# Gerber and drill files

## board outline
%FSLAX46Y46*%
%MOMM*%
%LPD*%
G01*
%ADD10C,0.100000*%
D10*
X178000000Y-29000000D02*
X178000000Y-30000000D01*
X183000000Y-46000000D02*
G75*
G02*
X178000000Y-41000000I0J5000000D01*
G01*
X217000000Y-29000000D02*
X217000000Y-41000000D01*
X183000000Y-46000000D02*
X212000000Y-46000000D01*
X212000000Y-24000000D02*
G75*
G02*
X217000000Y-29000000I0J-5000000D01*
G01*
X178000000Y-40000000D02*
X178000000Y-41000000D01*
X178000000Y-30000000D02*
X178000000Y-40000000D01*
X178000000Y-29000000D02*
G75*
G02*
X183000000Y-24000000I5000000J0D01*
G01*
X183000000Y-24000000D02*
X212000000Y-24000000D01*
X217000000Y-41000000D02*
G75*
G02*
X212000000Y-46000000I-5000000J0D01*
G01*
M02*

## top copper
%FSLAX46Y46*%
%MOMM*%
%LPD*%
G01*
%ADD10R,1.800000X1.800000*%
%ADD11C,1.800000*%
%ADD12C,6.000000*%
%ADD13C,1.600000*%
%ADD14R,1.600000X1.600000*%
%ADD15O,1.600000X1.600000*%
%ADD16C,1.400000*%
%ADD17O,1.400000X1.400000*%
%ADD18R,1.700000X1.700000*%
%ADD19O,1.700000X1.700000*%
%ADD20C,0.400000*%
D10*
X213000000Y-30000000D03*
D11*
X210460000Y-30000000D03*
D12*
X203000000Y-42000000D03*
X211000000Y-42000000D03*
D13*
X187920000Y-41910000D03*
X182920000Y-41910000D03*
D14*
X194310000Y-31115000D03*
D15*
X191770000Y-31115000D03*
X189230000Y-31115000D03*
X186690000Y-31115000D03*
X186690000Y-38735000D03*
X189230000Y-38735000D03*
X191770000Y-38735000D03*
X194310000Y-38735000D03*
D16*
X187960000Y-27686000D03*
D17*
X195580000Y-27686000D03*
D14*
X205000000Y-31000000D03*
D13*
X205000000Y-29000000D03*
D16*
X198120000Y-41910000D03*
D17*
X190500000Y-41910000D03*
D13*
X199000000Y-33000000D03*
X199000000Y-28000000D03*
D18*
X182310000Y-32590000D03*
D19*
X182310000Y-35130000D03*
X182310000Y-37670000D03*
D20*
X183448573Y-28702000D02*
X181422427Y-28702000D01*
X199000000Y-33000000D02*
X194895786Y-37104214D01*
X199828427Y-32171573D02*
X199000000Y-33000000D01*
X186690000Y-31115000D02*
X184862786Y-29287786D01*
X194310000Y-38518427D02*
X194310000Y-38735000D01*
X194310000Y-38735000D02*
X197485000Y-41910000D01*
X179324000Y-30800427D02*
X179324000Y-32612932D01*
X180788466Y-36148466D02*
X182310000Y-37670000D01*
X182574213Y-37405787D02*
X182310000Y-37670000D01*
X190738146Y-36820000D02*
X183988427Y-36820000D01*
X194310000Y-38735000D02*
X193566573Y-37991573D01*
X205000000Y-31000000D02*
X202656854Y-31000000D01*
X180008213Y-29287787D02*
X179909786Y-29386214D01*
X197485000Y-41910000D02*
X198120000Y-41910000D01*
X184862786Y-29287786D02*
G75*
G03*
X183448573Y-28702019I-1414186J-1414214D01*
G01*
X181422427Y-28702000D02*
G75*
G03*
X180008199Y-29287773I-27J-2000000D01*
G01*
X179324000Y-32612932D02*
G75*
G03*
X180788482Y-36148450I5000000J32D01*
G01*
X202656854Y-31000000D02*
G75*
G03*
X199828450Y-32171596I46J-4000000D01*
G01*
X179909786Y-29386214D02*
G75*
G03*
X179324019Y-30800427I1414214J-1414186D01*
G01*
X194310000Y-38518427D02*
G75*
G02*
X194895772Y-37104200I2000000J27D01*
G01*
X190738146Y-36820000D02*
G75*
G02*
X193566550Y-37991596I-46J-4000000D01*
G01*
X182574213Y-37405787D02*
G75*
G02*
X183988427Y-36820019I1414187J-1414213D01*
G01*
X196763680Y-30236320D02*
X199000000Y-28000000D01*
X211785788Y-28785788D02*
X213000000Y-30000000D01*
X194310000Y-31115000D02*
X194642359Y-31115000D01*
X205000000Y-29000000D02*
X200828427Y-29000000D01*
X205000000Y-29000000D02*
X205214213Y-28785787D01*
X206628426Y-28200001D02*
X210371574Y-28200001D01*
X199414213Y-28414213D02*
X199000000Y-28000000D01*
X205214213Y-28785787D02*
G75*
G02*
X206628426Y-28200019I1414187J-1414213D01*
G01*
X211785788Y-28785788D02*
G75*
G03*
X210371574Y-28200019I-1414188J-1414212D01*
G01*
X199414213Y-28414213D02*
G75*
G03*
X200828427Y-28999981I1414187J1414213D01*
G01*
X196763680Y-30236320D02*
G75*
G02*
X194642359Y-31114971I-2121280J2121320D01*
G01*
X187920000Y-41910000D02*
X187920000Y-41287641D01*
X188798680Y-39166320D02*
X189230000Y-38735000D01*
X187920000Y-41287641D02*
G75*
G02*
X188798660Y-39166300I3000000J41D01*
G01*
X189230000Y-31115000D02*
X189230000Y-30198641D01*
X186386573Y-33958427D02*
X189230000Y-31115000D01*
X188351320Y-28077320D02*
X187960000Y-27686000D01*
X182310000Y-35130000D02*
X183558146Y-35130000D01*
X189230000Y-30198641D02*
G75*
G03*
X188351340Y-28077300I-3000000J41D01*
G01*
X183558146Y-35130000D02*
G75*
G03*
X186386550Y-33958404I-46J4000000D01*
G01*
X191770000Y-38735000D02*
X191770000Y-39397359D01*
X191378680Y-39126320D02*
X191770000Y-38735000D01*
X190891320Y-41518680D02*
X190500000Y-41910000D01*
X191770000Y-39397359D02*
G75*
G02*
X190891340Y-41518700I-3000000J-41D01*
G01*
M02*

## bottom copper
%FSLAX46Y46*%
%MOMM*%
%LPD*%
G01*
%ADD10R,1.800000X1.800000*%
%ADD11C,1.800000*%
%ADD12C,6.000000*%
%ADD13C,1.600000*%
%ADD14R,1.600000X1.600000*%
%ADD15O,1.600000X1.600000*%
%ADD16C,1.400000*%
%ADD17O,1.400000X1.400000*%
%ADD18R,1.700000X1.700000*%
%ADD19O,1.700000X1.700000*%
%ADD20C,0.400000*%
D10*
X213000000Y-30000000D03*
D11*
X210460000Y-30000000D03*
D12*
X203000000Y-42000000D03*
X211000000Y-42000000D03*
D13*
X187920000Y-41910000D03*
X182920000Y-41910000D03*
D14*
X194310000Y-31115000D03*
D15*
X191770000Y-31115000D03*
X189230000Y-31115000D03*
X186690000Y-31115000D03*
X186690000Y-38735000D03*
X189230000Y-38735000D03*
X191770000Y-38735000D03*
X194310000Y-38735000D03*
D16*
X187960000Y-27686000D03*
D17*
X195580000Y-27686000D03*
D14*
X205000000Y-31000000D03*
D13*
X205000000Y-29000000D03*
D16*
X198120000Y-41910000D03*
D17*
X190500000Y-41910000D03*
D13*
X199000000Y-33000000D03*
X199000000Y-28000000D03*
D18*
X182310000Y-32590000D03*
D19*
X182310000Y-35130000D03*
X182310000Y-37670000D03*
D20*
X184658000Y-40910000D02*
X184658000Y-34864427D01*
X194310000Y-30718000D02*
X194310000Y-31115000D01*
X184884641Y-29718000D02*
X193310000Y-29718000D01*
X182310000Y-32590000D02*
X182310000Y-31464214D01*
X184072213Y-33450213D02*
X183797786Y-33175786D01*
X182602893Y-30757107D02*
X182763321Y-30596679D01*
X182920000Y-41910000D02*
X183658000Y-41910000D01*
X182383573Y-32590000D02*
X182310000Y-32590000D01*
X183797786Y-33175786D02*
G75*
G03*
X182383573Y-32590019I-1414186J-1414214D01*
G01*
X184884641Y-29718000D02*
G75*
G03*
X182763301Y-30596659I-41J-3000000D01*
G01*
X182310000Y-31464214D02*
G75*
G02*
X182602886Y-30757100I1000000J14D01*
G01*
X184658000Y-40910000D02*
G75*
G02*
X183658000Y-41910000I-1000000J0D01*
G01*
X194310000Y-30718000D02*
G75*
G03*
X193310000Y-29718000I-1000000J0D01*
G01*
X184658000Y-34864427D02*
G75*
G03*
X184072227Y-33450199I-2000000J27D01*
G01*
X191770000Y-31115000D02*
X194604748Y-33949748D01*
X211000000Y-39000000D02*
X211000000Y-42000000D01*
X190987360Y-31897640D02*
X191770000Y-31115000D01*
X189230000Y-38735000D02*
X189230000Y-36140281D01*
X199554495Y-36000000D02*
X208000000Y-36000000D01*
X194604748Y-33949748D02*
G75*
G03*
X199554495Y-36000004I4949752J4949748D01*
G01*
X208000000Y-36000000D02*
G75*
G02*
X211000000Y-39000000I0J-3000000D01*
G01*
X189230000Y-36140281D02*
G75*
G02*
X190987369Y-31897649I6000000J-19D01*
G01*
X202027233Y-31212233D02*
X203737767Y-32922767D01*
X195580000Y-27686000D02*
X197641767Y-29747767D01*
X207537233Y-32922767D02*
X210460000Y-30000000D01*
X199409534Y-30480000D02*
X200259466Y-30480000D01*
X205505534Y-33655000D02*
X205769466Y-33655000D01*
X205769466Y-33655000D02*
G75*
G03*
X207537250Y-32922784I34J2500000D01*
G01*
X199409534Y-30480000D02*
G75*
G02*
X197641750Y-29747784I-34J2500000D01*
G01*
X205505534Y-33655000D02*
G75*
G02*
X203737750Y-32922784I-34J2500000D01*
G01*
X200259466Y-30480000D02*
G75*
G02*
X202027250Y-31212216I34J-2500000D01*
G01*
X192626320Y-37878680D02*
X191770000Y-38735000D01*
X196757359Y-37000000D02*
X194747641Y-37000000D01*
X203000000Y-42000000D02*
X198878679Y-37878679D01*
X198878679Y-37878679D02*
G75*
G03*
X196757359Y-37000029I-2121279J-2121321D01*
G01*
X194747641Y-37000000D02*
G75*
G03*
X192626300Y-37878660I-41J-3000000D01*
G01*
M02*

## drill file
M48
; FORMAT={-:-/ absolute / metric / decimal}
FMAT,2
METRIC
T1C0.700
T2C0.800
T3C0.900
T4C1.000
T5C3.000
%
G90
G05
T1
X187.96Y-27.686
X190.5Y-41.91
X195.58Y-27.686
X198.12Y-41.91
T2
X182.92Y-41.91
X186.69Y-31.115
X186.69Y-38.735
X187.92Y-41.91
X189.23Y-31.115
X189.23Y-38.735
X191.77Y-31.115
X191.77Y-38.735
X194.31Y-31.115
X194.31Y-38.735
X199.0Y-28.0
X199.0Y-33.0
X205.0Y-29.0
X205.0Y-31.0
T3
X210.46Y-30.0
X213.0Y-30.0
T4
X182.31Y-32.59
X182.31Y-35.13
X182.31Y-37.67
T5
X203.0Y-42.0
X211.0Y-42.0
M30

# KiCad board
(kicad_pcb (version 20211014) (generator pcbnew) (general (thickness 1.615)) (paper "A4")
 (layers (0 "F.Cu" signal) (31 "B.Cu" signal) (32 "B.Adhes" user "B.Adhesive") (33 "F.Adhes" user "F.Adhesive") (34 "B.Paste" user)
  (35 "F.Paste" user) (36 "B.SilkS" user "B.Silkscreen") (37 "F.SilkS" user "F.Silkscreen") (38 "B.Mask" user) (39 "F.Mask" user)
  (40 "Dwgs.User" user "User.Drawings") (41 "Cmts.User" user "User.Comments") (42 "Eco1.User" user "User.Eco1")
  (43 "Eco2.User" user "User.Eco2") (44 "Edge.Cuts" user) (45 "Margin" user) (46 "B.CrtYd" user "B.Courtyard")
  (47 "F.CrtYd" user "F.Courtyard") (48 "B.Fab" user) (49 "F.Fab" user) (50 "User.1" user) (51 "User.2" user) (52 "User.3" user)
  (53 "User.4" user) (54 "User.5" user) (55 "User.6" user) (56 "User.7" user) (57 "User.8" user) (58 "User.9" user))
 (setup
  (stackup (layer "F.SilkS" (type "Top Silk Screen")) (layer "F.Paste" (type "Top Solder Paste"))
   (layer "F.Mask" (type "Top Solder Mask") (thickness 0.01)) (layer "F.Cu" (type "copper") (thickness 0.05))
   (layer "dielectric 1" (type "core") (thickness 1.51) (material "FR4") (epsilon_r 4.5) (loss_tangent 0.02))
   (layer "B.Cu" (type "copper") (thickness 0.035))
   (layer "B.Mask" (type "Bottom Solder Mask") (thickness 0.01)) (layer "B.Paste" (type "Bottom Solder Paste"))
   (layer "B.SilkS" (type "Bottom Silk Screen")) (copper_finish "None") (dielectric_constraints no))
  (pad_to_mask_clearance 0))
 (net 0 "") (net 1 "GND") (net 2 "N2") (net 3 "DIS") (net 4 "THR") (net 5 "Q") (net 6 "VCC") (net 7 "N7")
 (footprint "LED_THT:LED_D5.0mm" (layer "F.Cu") (at 213 30 180)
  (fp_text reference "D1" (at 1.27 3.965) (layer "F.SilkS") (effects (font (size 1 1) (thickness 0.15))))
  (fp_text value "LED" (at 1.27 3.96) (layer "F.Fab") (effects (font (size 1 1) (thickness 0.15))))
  (pad "1" thru_hole rect (at 0 0 180) (size 1.8 1.8) (drill 0.9) (layers *.Cu *.Mask) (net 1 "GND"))
  (pad "2" thru_hole circle (at 2.54 0 180) (size 1.8 1.8) (drill 0.9) (layers *.Cu *.Mask) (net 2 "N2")))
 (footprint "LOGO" (layer "F.Cu") (at 188 34.75)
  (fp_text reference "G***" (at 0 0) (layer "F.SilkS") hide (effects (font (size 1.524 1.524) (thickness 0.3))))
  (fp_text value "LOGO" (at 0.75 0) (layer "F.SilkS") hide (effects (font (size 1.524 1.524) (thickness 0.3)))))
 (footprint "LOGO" (layer "F.Cu") (at 183.896 28.575)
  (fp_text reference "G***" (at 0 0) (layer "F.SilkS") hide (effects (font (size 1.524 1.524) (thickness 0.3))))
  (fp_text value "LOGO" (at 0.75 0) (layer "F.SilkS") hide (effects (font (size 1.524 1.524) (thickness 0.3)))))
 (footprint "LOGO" (layer "F.Cu") (at 186 34.75)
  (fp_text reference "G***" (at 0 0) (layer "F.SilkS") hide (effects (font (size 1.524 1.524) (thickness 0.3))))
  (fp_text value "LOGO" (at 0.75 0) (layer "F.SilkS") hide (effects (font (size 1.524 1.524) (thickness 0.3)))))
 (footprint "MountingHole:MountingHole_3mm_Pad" (layer "F.Cu") (at 203 42)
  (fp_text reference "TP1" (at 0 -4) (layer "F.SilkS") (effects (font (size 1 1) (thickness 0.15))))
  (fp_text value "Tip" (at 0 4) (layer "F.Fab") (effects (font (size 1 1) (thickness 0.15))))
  (pad "1" thru_hole circle (at 0 0) (size 6 6) (drill 3) (layers *.Cu *.Mask) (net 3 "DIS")))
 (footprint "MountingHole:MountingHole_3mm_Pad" (layer "F.Cu") (at 211 42)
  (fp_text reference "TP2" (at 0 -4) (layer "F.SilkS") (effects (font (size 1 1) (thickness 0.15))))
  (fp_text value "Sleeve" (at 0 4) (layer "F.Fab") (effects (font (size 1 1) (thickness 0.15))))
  (pad "1" thru_hole circle (at 0 0) (size 6 6) (drill 3) (layers *.Cu *.Mask) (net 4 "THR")))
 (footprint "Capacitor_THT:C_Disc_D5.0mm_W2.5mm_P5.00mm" (layer "F.Cu") (at 187.92 41.91 180)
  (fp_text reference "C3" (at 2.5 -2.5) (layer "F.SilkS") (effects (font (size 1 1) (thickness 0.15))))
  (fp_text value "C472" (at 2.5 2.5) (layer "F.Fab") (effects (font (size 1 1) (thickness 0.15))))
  (pad "1" thru_hole circle (at 0 0 180) (size 1.6 1.6) (drill 0.8) (layers *.Cu *.Mask) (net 4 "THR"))
  (pad "2" thru_hole circle (at 5 0 180) (size 1.6 1.6) (drill 0.8) (layers *.Cu *.Mask) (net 1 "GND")))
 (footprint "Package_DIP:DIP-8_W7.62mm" (layer "F.Cu") (at 194.31 31.115 -90)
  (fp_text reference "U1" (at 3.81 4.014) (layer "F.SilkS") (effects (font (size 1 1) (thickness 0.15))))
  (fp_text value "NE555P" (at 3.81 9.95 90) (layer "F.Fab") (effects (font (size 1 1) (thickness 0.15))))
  (pad "1" thru_hole rect (at 0 0 270) (size 1.6 1.6) (drill 0.8) (layers *.Cu *.Mask) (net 1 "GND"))
  (pad "2" thru_hole oval (at 0 2.54 270) (size 1.6 1.6) (drill 0.8) (layers *.Cu *.Mask) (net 4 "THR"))
  (pad "3" thru_hole oval (at 0 5.08 270) (size 1.6 1.6) (drill 0.8) (layers *.Cu *.Mask) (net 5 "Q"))
  (pad "4" thru_hole oval (at 0 7.62 270) (size 1.6 1.6) (drill 0.8) (layers *.Cu *.Mask) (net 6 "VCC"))
  (pad "5" thru_hole oval (at 7.62 7.62 270) (size 1.6 1.6) (drill 0.8) (layers *.Cu *.Mask) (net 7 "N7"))
  (pad "6" thru_hole oval (at 7.62 5.08 270) (size 1.6 1.6) (drill 0.8) (layers *.Cu *.Mask) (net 4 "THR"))
  (pad "7" thru_hole oval (at 7.62 2.54 270) (size 1.6 1.6) (drill 0.8) (layers *.Cu *.Mask) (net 3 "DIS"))
  (pad "8" thru_hole oval (at 7.62 0 270) (size 1.6 1.6) (drill 0.8) (layers *.Cu *.Mask) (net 6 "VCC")))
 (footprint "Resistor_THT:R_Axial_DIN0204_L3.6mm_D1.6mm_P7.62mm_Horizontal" (layer "F.Cu") (at 187.96 27.686)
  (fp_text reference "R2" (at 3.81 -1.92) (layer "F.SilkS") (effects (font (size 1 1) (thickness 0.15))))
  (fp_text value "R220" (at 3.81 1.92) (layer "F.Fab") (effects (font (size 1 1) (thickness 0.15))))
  (pad "1" thru_hole circle (at 0 0) (size 1.4 1.4) (drill 0.7) (layers *.Cu *.Mask) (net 5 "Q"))
  (pad "2" thru_hole oval (at 7.62 0) (size 1.4 1.4) (drill 0.7) (layers *.Cu *.Mask) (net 2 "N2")))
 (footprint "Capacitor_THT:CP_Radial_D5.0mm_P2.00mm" (layer "F.Cu") (at 205 31 90)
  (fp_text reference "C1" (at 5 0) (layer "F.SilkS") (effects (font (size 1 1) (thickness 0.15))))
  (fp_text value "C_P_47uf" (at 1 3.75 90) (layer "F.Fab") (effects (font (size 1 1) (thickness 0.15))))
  (pad "1" thru_hole rect (at 0 0 90) (size 1.6 1.6) (drill 0.8) (layers *.Cu *.Mask) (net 6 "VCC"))
  (pad "2" thru_hole circle (at 2 0 90) (size 1.6 1.6) (drill 0.8) (layers *.Cu *.Mask) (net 1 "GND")))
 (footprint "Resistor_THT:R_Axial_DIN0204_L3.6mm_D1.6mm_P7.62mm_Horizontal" (layer "F.Cu") (at 198.12 41.91 180)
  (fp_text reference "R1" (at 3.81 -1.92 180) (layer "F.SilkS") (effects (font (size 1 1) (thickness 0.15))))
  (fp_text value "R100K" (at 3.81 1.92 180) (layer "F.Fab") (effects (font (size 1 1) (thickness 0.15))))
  (pad "1" thru_hole circle (at 0 0 180) (size 1.4 1.4) (drill 0.7) (layers *.Cu *.Mask) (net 6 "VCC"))
  (pad "2" thru_hole oval (at 7.62 0 180) (size 1.4 1.4) (drill 0.7) (layers *.Cu *.Mask) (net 3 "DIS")))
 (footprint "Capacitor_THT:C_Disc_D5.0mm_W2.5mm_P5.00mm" (layer "F.Cu") (at 199 33 90)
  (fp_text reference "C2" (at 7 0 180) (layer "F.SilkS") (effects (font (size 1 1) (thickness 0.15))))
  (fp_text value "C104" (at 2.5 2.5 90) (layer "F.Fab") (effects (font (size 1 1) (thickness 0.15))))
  (pad "1" thru_hole circle (at 0 0 90) (size 1.6 1.6) (drill 0.8) (layers *.Cu *.Mask) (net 6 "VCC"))
  (pad "2" thru_hole circle (at 5 0 90) (size 1.6 1.6) (drill 0.8) (layers *.Cu *.Mask) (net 1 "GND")))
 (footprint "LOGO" (layer "F.Cu") (at 181.864 28.575)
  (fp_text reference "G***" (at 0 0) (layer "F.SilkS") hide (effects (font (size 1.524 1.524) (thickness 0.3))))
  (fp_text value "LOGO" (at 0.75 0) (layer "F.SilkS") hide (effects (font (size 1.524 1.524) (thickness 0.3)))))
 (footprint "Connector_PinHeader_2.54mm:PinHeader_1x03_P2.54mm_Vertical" (layer "F.Cu") (at 182.31 32.59)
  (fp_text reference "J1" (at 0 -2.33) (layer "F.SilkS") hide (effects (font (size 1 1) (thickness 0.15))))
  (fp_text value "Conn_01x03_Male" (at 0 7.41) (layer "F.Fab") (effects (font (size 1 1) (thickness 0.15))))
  (pad "1" thru_hole rect (at 0 0) (size 1.7 1.7) (drill 1) (layers *.Cu *.Mask) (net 1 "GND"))
  (pad "2" thru_hole oval (at 0 2.54) (size 1.7 1.7) (drill 1) (layers *.Cu *.Mask) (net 5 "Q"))
  (pad "3" thru_hole oval (at 0 5.08) (size 1.7 1.7) (drill 1) (layers *.Cu *.Mask) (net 6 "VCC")))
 (gr_line (start 178 29) (end 178 30) (layer "Edge.Cuts") (width 0.1))
 (gr_arc (start 183 46) (mid 179.464466 44.535534) (end 178 41) (layer "Edge.Cuts") (width 0.1))
 (gr_line (start 217 29) (end 217 41) (layer "Edge.Cuts") (width 0.1))
 (gr_line (start 183 46) (end 212 46) (layer "Edge.Cuts") (width 0.1))
 (gr_arc (start 212 24) (mid 215.535534 25.464466) (end 217 29) (layer "Edge.Cuts") (width 0.1))
 (gr_line (start 178 40) (end 178 41) (layer "Edge.Cuts") (width 0.1))
 (gr_line (start 178 30) (end 178 40) (layer "Edge.Cuts") (width 0.1))
 (gr_arc (start 178 29) (mid 179.464466 25.464466) (end 183 24) (layer "Edge.Cuts") (width 0.1))
 (gr_line (start 183 24) (end 212 24) (layer "Edge.Cuts") (width 0.1))
 (gr_arc (start 217 41) (mid 215.535534 44.535534) (end 212 46) (layer "Edge.Cuts") (width 0.1))
 (segment (start 183.448573 28.702) (end 181.422427 28.702) (width 0.4) (layer "F.Cu") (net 6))
 (segment (start 199 33) (end 194.895786 37.104214) (width 0.4) (layer "F.Cu") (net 6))
 (segment (start 199.828427 32.171573) (end 199 33) (width 0.4) (layer "F.Cu") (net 6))
 (segment (start 186.69 31.115) (end 184.862786 29.287786) (width 0.4) (layer "F.Cu") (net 6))
 (segment (start 194.31 38.518427) (end 194.31 38.735) (width 0.4) (layer "F.Cu") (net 6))
 (segment (start 194.31 38.735) (end 197.485 41.91) (width 0.4) (layer "F.Cu") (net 6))
 (segment (start 179.324 30.800427) (end 179.324 32.612932) (width 0.4) (layer "F.Cu") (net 6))
 (segment (start 180.788466 36.148466) (end 182.31 37.67) (width 0.4) (layer "F.Cu") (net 6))
 (segment (start 182.574213 37.405787) (end 182.31 37.67) (width 0.4) (layer "F.Cu") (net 6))
 (segment (start 190.738146 36.82) (end 183.988427 36.82) (width 0.4) (layer "F.Cu") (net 6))
 (segment (start 194.31 38.735) (end 193.566573 37.991573) (width 0.4) (layer "F.Cu") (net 6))
 (segment (start 205 31) (end 202.656854 31) (width 0.4) (layer "F.Cu") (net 6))
 (segment (start 180.008213 29.287787) (end 179.909786 29.386214) (width 0.4) (layer "F.Cu") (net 6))
 (segment (start 197.485 41.91) (end 198.12 41.91) (width 0.4) (layer "F.Cu") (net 6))
 (arc (start 184.862786 29.287786) (mid 184.21394 28.854241) (end 183.448573 28.702) (width 0.4) (layer "F.Cu") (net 6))
 (arc (start 181.422427 28.702) (mid 180.65706 28.854241) (end 180.008213 29.287787) (width 0.4) (layer "F.Cu") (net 6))
 (arc (start 179.324 32.612932) (mid 179.704602 34.526349) (end 180.788466 36.148466) (width 0.4) (layer "F.Cu") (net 6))
 (arc (start 202.656854 31) (mid 201.12612 31.304482) (end 199.828427 32.171573) (width 0.4) (layer "F.Cu") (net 6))
 (arc (start 179.909786 29.386214) (mid 179.476241 30.03506) (end 179.324 30.800427) (width 0.4) (layer "F.Cu") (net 6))
 (arc (start 194.31 38.518427) (mid 194.462241 37.75306) (end 194.895786 37.104214) (width 0.4) (layer "F.Cu") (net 6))
 (arc (start 190.738146 36.82) (mid 192.26888 37.124482) (end 193.566573 37.991573) (width 0.4) (layer "F.Cu") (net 6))
 (arc (start 182.574213 37.405787) (mid 183.22306 36.972241) (end 183.988427 36.82) (width 0.4) (layer "F.Cu") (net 6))
 (segment (start 196.76368 30.23632) (end 199 28) (width 0.4) (layer "F.Cu") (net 1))
 (segment (start 211.785788 28.785788) (end 213 30) (width 0.4) (layer "F.Cu") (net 1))
 (segment (start 194.31 31.115) (end 194.642359 31.115) (width 0.4) (layer "F.Cu") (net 1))
 (segment (start 205 29) (end 200.828427 29) (width 0.4) (layer "F.Cu") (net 1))
 (segment (start 205 29) (end 205.214213 28.785787) (width 0.4) (layer "F.Cu") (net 1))
 (segment (start 206.628426 28.200001) (end 210.371574 28.200001) (width 0.4) (layer "F.Cu") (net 1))
 (segment (start 199.414213 28.414213) (end 199 28) (width 0.4) (layer "F.Cu") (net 1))
 (arc (start 205.214213 28.785787) (mid 205.863059 28.352242) (end 206.628426 28.200001) (width 0.4) (layer "F.Cu") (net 1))
 (arc (start 211.785788 28.785788) (mid 211.136941 28.352242) (end 210.371574 28.200001) (width 0.4) (layer "F.Cu") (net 1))
 (arc (start 199.414213 28.414213) (mid 200.06306 28.847759) (end 200.828427 29) (width 0.4) (layer "F.Cu") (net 1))
 (arc (start 196.76368 30.23632) (mid 195.79041 30.886639) (end 194.642359 31.115) (width 0.4) (layer "F.Cu") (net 1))
 (segment (start 184.658 40.91) (end 184.658 34.864427) (width 0.4) (layer "B.Cu") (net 1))
 (segment (start 194.31 30.718) (end 194.31 31.115) (width 0.4) (layer "B.Cu") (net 1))
 (segment (start 184.884641 29.718) (end 193.31 29.718) (width 0.4) (layer "B.Cu") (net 1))
 (segment (start 182.31 32.59) (end 182.31 31.464214) (width 0.4) (layer "B.Cu") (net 1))
 (segment (start 184.072213 33.450213) (end 183.797786 33.175786) (width 0.4) (layer "B.Cu") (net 1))
 (segment (start 182.602893 30.757107) (end 182.763321 30.596679) (width 0.4) (layer "B.Cu") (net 1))
 (segment (start 182.92 41.91) (end 183.658 41.91) (width 0.4) (layer "B.Cu") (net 1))
 (segment (start 182.383573 32.59) (end 182.31 32.59) (width 0.4) (layer "B.Cu") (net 1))
 (arc (start 183.797786 33.175786) (mid 183.14894 32.742241) (end 182.383573 32.59) (width 0.4) (layer "B.Cu") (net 1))
 (arc (start 184.884641 29.718) (mid 183.736591 29.946361) (end 182.763321 30.596679) (width 0.4) (layer "B.Cu") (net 1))
 (arc (start 182.31 31.464214) (mid 182.38612 31.081531) (end 182.602893 30.757107) (width 0.4) (layer "B.Cu") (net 1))
 (arc (start 184.658 40.91) (mid 184.365107 41.617107) (end 183.658 41.91) (width 0.4) (layer "B.Cu") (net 1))
 (arc (start 194.31 30.718) (mid 194.017107 30.010893) (end 193.31 29.718) (width 0.4) (layer "B.Cu") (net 1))
 (arc (start 184.658 34.864427) (mid 184.505759 34.09906) (end 184.072213 33.450213) (width 0.4) (layer "B.Cu") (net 1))
 (segment (start 187.92 41.91) (end 187.92 41.287641) (width 0.4) (layer "F.Cu") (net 4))
 (segment (start 188.79868 39.16632) (end 189.23 38.735) (width 0.4) (layer "F.Cu") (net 4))
 (arc (start 187.92 41.287641) (mid 188.148362 40.13959) (end 188.79868 39.16632) (width 0.4) (layer "F.Cu") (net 4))
 (segment (start 191.77 31.115) (end 194.604748 33.949748) (width 0.4) (layer "B.Cu") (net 4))
 (segment (start 211 39) (end 211 42) (width 0.4) (layer "B.Cu") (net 4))
 (segment (start 190.98736 31.89764) (end 191.77 31.115) (width 0.4) (layer "B.Cu") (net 4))
 (segment (start 189.23 38.735) (end 189.23 36.140281) (width 0.4) (layer "B.Cu") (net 4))
 (segment (start 199.554495 36) (end 208 36) (width 0.4) (layer "B.Cu") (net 4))
 (arc (start 194.604748 33.949748) (mid 196.875711 35.467157) (end 199.554495 36) (width 0.4) (layer "B.Cu") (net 4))
 (arc (start 208 36) (mid 210.12132 36.87868) (end 211 39) (width 0.4) (layer "B.Cu") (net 4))
 (arc (start 189.23 36.140281) (mid 189.686723 33.84418) (end 190.98736 31.89764) (width 0.4) (layer "B.Cu") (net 4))
 (segment (start 202.027233 31.212233) (end 203.737767 32.922767) (width 0.4) (layer "B.Cu") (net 2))
 (segment (start 195.58 27.686) (end 197.641767 29.747767) (width 0.4) (layer "B.Cu") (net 2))
 (segment (start 207.537233 32.922767) (end 210.46 30) (width 0.4) (layer "B.Cu") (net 2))
 (segment (start 199.409534 30.48) (end 200.259466 30.48) (width 0.4) (layer "B.Cu") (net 2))
 (segment (start 205.505534 33.655) (end 205.769466 33.655) (width 0.4) (layer "B.Cu") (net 2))
 (arc (start 205.769466 33.655) (mid 206.726175 33.464699) (end 207.537233 32.922767) (width 0.4) (layer "B.Cu") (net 2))
 (arc (start 199.409534 30.48) (mid 198.452825 30.289699) (end 197.641767 29.747767) (width 0.4) (layer "B.Cu") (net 2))
 (arc (start 205.505534 33.655) (mid 204.548825 33.464699) (end 203.737767 32.922767) (width 0.4) (layer "B.Cu") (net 2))
 (arc (start 200.259466 30.48) (mid 201.216175 30.670301) (end 202.027233 31.212233) (width 0.4) (layer "B.Cu") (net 2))
 (segment (start 189.23 31.115) (end 189.23 30.198641) (width 0.4) (layer "F.Cu") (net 5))
 (segment (start 186.386573 33.958427) (end 189.23 31.115) (width 0.4) (layer "F.Cu") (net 5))
 (segment (start 188.35132 28.07732) (end 187.96 27.686) (width 0.4) (layer "F.Cu") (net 5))
 (segment (start 182.31 35.13) (end 183.558146 35.13) (width 0.4) (layer "F.Cu") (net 5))
 (arc (start 189.23 30.198641) (mid 189.001638 29.05059) (end 188.35132 28.07732) (width 0.4) (layer "F.Cu") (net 5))
 (arc (start 183.558146 35.13) (mid 185.08888 34.825518) (end 186.386573 33.958427) (width 0.4) (layer "F.Cu") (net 5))
 (segment (start 191.77 38.735) (end 191.77 39.397359) (width 0.4) (layer "F.Cu") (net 3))
 (segment (start 191.37868 39.12632) (end 191.77 38.735) (width 0.4) (layer "F.Cu") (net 3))
 (segment (start 190.89132 41.51868) (end 190.5 41.91) (width 0.4) (layer "F.Cu") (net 3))
 (arc (start 191.77 39.397359) (mid 191.541638 40.54541) (end 190.89132 41.51868) (width 0.4) (layer "F.Cu") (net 3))
 (segment (start 192.62632 37.87868) (end 191.77 38.735) (width 0.4) (layer "B.Cu") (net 3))
 (segment (start 196.757359 37) (end 194.747641 37) (width 0.4) (layer "B.Cu") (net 3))
 (segment (start 203 42) (end 198.878679 37.878679) (width 0.4) (layer "B.Cu") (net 3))
 (arc (start 198.878679 37.878679) (mid 197.905409 37.228361) (end 196.757359 37) (width 0.4) (layer "B.Cu") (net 3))
 (arc (start 194.747641 37) (mid 193.59959 37.228362) (end 192.62632 37.87868) (width 0.4) (layer "B.Cu") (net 3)))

